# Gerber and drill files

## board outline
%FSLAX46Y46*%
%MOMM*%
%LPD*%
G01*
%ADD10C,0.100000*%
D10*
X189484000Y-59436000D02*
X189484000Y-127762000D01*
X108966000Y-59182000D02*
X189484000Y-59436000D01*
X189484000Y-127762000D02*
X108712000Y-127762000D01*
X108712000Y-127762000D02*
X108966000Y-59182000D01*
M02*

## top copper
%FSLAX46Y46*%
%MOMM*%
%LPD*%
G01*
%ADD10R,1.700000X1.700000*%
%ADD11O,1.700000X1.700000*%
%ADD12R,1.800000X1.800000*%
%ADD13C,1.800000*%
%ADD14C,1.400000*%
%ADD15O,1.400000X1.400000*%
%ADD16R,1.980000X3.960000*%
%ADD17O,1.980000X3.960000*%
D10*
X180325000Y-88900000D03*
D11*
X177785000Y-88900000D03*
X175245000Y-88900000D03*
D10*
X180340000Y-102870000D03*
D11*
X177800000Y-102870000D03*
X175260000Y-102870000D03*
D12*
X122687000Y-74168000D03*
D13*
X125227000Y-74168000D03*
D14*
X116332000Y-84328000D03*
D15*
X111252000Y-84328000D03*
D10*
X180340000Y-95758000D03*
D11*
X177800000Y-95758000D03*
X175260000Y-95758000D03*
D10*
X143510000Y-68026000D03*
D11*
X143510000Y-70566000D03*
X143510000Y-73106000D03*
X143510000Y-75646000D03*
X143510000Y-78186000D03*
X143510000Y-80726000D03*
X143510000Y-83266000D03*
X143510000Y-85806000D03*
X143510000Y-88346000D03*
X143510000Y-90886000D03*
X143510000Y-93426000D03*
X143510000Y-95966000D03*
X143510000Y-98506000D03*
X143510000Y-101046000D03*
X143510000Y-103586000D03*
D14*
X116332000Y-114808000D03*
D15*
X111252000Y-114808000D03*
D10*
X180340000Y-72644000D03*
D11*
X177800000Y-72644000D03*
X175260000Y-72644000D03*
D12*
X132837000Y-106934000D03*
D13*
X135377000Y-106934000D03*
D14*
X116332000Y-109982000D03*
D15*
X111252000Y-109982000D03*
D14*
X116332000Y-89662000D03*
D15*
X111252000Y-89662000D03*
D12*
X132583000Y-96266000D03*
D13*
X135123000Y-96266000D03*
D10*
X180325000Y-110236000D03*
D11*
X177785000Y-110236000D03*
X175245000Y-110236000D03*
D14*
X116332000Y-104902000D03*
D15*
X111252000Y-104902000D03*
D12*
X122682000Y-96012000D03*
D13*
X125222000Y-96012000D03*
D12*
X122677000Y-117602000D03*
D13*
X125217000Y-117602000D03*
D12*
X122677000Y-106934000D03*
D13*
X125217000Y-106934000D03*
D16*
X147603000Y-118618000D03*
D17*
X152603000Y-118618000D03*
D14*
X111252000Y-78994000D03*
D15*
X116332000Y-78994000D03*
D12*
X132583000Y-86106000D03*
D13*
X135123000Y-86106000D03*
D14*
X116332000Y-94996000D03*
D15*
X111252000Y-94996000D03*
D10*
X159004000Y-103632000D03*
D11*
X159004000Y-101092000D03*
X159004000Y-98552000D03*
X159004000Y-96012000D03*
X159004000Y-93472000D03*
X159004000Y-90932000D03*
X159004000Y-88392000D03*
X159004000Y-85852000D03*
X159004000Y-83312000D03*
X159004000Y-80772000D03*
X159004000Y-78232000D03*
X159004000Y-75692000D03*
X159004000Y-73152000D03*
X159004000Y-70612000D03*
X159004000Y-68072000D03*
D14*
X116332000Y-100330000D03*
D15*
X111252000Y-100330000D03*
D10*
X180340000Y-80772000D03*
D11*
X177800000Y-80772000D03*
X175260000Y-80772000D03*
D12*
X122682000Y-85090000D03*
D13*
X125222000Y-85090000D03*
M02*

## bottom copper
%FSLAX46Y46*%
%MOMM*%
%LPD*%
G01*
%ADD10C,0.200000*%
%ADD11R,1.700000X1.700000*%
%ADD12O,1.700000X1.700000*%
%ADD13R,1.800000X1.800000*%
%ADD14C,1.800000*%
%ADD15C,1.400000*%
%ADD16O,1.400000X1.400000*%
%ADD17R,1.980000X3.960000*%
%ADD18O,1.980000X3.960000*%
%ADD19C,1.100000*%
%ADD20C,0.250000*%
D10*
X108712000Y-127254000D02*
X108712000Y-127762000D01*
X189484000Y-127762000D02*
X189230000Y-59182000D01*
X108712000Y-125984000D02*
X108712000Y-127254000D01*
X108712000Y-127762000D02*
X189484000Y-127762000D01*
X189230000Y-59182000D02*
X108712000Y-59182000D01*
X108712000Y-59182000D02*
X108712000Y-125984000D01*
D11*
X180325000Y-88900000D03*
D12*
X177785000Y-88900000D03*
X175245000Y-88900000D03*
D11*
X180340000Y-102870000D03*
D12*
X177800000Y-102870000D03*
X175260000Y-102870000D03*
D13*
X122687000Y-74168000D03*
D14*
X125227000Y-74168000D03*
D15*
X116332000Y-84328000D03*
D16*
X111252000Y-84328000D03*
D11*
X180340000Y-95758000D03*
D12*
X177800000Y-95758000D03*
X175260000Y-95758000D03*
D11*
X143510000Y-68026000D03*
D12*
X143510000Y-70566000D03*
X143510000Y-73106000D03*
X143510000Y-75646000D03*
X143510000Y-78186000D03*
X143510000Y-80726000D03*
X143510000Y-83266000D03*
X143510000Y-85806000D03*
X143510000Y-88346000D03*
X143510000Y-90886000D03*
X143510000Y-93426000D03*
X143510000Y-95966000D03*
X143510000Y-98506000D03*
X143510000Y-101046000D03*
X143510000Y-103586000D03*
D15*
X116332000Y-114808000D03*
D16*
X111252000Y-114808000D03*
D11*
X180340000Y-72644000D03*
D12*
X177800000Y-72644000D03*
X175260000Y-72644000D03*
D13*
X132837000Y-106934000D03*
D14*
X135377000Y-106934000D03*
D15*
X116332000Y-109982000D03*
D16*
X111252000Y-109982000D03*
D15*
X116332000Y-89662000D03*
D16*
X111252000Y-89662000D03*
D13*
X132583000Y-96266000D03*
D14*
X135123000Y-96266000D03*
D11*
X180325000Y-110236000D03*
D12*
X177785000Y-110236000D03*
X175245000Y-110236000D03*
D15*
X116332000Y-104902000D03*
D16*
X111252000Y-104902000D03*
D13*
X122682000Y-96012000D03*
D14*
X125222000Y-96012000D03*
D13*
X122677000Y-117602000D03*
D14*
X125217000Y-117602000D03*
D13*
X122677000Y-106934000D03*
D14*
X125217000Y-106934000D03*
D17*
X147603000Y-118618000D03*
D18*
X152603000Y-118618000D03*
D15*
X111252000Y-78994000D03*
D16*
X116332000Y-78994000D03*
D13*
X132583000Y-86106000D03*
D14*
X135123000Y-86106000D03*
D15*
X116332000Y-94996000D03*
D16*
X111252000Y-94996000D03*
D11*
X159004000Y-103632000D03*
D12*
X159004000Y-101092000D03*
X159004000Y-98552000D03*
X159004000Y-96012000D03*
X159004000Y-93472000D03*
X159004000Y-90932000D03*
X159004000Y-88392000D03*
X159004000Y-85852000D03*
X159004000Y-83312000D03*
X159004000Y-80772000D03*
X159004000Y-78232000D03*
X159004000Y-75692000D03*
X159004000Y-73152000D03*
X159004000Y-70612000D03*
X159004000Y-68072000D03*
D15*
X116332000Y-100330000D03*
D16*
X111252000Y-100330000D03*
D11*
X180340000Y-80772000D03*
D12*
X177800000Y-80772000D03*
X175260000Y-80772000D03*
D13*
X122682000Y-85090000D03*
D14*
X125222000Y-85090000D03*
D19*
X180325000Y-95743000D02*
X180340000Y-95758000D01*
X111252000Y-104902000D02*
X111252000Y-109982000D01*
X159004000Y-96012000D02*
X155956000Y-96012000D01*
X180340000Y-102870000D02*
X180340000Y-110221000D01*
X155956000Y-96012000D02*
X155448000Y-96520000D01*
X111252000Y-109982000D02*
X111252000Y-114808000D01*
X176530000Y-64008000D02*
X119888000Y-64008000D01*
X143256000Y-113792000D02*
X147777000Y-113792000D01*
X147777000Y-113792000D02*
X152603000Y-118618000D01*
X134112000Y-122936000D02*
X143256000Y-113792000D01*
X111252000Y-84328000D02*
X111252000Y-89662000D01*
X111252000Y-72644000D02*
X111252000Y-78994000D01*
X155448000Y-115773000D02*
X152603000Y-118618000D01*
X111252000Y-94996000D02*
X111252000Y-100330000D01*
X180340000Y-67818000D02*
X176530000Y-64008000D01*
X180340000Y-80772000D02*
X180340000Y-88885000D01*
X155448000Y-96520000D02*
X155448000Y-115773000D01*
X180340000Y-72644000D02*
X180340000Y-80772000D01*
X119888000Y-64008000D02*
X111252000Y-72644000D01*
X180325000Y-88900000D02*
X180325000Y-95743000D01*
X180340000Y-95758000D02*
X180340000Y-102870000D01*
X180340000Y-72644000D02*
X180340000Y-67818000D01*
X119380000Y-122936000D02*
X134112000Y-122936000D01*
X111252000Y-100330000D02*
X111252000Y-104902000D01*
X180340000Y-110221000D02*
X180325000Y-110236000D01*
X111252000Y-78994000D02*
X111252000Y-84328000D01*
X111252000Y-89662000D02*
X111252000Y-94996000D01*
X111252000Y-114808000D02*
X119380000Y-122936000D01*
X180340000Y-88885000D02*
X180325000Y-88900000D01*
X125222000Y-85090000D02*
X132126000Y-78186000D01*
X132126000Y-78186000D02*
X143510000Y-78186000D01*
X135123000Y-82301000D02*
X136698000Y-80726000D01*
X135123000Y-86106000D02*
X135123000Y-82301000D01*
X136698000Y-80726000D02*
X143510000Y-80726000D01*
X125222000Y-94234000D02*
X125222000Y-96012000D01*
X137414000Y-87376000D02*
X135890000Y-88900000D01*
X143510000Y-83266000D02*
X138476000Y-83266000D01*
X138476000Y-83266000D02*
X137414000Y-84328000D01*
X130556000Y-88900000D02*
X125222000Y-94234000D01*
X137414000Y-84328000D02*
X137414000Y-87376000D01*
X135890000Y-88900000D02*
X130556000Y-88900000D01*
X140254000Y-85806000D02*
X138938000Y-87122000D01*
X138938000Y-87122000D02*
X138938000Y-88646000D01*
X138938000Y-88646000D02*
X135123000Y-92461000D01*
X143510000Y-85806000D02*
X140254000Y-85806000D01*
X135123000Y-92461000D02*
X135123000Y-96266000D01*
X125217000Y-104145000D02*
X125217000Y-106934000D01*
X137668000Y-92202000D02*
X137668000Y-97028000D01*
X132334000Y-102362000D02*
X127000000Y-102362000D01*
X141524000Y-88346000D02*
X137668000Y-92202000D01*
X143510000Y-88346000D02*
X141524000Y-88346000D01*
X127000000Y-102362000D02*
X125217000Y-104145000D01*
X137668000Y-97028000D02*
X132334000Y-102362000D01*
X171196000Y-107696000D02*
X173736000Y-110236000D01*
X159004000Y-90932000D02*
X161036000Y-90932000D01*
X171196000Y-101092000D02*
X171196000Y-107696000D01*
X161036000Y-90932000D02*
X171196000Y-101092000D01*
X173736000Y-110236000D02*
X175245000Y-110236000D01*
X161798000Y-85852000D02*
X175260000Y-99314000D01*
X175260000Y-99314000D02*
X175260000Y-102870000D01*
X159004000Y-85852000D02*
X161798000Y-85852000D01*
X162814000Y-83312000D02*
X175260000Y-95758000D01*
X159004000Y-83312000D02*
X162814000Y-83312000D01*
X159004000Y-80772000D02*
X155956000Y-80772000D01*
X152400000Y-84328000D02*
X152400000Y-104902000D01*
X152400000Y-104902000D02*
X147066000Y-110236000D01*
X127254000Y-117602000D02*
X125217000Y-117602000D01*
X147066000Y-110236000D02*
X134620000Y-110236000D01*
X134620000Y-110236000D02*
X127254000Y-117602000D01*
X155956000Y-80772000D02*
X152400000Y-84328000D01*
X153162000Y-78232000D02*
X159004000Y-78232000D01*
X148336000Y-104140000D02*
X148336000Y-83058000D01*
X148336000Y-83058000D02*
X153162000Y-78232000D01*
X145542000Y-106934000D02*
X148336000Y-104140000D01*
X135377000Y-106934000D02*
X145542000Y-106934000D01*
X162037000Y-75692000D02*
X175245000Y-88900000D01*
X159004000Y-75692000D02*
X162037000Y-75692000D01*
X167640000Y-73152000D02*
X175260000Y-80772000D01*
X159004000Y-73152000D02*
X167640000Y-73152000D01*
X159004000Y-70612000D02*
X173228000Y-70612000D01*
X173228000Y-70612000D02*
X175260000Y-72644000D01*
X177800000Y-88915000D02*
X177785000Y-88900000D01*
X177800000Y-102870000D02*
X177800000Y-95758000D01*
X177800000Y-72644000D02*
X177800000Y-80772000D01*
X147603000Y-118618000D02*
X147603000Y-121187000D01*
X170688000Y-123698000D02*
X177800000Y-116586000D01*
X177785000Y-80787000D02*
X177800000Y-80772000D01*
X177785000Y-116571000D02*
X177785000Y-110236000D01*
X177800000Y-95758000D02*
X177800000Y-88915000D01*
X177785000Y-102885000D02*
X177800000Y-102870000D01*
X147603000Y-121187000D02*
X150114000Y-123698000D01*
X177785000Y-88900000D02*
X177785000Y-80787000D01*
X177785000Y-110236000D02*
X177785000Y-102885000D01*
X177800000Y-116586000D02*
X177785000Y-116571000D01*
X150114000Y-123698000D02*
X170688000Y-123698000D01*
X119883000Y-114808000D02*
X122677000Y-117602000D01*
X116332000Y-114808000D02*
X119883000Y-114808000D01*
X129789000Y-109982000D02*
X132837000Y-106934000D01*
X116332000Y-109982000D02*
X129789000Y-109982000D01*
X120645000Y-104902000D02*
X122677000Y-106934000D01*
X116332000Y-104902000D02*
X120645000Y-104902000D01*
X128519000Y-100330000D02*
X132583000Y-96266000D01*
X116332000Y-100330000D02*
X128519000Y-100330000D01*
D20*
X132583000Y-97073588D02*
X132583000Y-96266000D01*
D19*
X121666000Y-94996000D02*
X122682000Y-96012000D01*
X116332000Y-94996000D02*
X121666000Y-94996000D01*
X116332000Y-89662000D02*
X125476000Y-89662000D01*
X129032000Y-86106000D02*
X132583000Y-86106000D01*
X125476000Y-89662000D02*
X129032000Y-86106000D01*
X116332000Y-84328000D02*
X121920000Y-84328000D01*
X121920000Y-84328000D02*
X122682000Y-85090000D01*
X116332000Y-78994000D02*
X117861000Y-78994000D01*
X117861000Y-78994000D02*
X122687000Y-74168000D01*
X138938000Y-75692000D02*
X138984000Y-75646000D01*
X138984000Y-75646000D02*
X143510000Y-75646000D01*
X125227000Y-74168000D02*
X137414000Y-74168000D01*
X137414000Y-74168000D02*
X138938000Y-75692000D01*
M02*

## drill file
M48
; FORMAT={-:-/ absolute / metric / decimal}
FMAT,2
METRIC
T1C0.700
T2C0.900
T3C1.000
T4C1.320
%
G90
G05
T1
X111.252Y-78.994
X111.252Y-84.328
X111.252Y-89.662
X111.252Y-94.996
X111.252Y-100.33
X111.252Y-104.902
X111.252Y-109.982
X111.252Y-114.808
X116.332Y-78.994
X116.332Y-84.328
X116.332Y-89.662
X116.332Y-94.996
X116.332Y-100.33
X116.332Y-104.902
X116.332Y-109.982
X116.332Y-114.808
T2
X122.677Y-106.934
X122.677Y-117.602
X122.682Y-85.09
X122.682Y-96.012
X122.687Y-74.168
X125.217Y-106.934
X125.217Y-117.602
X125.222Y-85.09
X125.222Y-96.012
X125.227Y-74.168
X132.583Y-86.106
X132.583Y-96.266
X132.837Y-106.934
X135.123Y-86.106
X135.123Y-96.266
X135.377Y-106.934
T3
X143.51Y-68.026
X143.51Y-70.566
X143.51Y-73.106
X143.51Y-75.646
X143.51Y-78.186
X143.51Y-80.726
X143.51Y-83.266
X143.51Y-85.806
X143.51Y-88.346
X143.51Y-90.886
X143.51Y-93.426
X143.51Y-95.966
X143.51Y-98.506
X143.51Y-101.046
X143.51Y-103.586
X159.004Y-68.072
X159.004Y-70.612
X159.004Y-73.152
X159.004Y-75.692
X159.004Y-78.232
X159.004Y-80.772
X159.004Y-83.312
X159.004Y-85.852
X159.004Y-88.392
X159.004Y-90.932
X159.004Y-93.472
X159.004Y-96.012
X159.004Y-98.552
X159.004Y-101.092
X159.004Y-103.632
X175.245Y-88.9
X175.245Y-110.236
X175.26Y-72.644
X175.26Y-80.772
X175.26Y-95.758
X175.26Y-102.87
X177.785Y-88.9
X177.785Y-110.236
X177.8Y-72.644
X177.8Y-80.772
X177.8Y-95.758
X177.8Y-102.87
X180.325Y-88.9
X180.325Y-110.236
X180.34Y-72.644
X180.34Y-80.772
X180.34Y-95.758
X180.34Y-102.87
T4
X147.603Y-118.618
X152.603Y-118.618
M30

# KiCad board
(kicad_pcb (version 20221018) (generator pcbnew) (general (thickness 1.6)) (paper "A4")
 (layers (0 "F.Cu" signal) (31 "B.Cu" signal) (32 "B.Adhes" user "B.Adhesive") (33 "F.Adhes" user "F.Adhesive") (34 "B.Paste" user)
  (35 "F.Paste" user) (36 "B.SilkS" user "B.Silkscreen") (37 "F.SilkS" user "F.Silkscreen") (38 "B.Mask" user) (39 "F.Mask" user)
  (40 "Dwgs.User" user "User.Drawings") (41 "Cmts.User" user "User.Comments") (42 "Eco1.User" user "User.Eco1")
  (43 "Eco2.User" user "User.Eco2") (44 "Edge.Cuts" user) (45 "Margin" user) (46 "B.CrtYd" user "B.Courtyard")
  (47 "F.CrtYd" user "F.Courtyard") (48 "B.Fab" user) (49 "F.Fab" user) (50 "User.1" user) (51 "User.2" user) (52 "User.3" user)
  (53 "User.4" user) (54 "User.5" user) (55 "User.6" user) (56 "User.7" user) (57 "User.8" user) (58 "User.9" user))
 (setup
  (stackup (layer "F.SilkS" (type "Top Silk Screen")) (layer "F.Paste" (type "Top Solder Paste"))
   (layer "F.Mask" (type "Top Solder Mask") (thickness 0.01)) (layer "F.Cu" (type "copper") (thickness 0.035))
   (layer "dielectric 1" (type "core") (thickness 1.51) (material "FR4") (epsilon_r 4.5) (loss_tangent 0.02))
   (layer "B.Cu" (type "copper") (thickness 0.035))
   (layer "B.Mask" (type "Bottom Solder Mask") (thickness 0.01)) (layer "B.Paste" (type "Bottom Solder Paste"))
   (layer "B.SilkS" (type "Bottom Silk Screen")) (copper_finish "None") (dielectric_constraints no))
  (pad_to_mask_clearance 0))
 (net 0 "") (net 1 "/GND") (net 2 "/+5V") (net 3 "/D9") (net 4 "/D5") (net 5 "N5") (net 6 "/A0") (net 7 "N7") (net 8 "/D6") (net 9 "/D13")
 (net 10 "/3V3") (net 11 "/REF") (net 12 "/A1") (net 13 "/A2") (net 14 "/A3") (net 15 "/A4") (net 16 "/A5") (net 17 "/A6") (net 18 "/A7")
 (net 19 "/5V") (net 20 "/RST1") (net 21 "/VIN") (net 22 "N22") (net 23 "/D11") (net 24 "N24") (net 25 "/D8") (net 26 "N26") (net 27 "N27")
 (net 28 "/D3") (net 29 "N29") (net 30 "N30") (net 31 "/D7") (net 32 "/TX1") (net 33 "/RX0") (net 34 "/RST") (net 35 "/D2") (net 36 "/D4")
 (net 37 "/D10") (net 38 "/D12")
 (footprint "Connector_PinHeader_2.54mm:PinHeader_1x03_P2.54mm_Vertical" (layer "F.Cu") (at 180.325 88.9 -90)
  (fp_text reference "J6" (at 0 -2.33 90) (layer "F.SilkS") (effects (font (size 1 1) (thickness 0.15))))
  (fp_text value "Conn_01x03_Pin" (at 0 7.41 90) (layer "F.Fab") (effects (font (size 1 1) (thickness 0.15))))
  (pad "1" thru_hole rect (at 0 0 270) (size 1.7 1.7) (drill 1) (layers "*.Cu" "*.Mask") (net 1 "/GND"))
  (pad "2" thru_hole oval (at 0 2.54 270) (size 1.7 1.7) (drill 1) (layers "*.Cu" "*.Mask") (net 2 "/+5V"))
  (pad "3" thru_hole oval (at 0 5.08 270) (size 1.7 1.7) (drill 1) (layers "*.Cu" "*.Mask") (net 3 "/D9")))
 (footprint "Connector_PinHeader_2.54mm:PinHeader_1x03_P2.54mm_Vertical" (layer "F.Cu") (at 180.34 102.87 -90)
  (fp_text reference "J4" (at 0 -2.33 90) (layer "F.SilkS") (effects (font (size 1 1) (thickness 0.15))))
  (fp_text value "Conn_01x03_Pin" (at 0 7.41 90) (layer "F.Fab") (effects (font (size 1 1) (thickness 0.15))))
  (pad "1" thru_hole rect (at 0 0 270) (size 1.7 1.7) (drill 1) (layers "*.Cu" "*.Mask") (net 1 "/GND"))
  (pad "2" thru_hole oval (at 0 2.54 270) (size 1.7 1.7) (drill 1) (layers "*.Cu" "*.Mask") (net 2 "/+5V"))
  (pad "3" thru_hole oval (at 0 5.08 270) (size 1.7 1.7) (drill 1) (layers "*.Cu" "*.Mask") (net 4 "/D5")))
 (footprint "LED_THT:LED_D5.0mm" (layer "F.Cu") (at 122.687 74.168)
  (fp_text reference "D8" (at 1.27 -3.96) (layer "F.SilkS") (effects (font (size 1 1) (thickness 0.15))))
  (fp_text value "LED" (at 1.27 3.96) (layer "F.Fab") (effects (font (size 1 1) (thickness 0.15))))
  (pad "1" thru_hole rect (at 0 0) (size 1.8 1.8) (drill 0.9) (layers "*.Cu" "*.Mask") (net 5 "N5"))
  (pad "2" thru_hole circle (at 2.54 0) (size 1.8 1.8) (drill 0.9) (layers "*.Cu" "*.Mask") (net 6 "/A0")))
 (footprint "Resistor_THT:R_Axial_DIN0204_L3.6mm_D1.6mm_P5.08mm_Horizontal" (layer "F.Cu") (at 116.332 84.328 180)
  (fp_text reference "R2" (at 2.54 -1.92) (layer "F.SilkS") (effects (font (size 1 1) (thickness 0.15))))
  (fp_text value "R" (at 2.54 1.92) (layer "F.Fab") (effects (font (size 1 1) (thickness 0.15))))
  (pad "1" thru_hole circle (at 0 0 180) (size 1.4 1.4) (drill 0.7) (layers "*.Cu" "*.Mask") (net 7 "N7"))
  (pad "2" thru_hole oval (at 5.08 0 180) (size 1.4 1.4) (drill 0.7) (layers "*.Cu" "*.Mask") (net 1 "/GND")))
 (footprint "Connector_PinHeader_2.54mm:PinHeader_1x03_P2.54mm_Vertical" (layer "F.Cu") (at 180.34 95.758 -90)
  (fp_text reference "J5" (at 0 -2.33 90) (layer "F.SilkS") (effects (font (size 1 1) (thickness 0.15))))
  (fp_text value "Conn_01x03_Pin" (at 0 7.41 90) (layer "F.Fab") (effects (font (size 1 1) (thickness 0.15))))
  (pad "1" thru_hole rect (at 0 0 270) (size 1.7 1.7) (drill 1) (layers "*.Cu" "*.Mask") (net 1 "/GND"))
  (pad "2" thru_hole oval (at 0 2.54 270) (size 1.7 1.7) (drill 1) (layers "*.Cu" "*.Mask") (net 2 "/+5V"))
  (pad "3" thru_hole oval (at 0 5.08 270) (size 1.7 1.7) (drill 1) (layers "*.Cu" "*.Mask") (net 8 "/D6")))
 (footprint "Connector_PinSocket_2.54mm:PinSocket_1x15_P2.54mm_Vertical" (layer "F.Cu") (at 143.51 68.026)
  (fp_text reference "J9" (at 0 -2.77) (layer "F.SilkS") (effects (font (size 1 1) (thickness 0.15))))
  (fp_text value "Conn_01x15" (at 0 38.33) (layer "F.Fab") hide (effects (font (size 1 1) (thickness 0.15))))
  (pad "1" thru_hole rect (at 0 0) (size 1.7 1.7) (drill 1) (layers "*.Cu" "*.Mask") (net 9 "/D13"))
  (pad "2" thru_hole oval (at 0 2.54) (size 1.7 1.7) (drill 1) (layers "*.Cu" "*.Mask") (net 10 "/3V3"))
  (pad "3" thru_hole oval (at 0 5.08) (size 1.7 1.7) (drill 1) (layers "*.Cu" "*.Mask") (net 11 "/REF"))
  (pad "4" thru_hole oval (at 0 7.62) (size 1.7 1.7) (drill 1) (layers "*.Cu" "*.Mask") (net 6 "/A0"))
  (pad "5" thru_hole oval (at 0 10.16) (size 1.7 1.7) (drill 1) (layers "*.Cu" "*.Mask") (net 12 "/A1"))
  (pad "6" thru_hole oval (at 0 12.7) (size 1.7 1.7) (drill 1) (layers "*.Cu" "*.Mask") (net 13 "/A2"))
  (pad "7" thru_hole oval (at 0 15.24) (size 1.7 1.7) (drill 1) (layers "*.Cu" "*.Mask") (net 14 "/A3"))
  (pad "8" thru_hole oval (at 0 17.78) (size 1.7 1.7) (drill 1) (layers "*.Cu" "*.Mask") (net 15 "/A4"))
  (pad "9" thru_hole oval (at 0 20.32) (size 1.7 1.7) (drill 1) (layers "*.Cu" "*.Mask") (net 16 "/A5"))
  (pad "10" thru_hole oval (at 0 22.86) (size 1.7 1.7) (drill 1) (layers "*.Cu" "*.Mask") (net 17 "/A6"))
  (pad "11" thru_hole oval (at 0 25.4) (size 1.7 1.7) (drill 1) (layers "*.Cu" "*.Mask") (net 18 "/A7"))
  (pad "12" thru_hole oval (at 0 27.94) (size 1.7 1.7) (drill 1) (layers "*.Cu" "*.Mask") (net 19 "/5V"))
  (pad "13" thru_hole oval (at 0 30.48) (size 1.7 1.7) (drill 1) (layers "*.Cu" "*.Mask") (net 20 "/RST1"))
  (pad "14" thru_hole oval (at 0 33.02) (size 1.7 1.7) (drill 1) (layers "*.Cu" "*.Mask") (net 1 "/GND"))
  (pad "15" thru_hole oval (at 0 35.56) (size 1.7 1.7) (drill 1) (layers "*.Cu" "*.Mask") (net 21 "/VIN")))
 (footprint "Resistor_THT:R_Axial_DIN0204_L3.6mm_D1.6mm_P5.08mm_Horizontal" (layer "F.Cu") (at 116.332 114.808 180)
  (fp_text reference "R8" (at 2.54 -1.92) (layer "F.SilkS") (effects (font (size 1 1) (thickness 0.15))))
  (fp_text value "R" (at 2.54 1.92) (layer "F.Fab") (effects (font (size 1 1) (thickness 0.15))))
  (pad "1" thru_hole circle (at 0 0 180) (size 1.4 1.4) (drill 0.7) (layers "*.Cu" "*.Mask") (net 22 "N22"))
  (pad "2" thru_hole oval (at 5.08 0 180) (size 1.4 1.4) (drill 0.7) (layers "*.Cu" "*.Mask") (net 1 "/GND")))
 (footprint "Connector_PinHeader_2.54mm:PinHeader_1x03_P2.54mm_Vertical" (layer "F.Cu") (at 180.34 72.644 -90)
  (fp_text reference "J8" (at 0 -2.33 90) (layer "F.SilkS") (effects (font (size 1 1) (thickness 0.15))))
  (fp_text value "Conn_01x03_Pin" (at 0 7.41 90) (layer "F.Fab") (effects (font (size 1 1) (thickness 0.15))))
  (pad "1" thru_hole rect (at 0 0 270) (size 1.7 1.7) (drill 1) (layers "*.Cu" "*.Mask") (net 1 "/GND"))
  (pad "2" thru_hole oval (at 0 2.54 270) (size 1.7 1.7) (drill 1) (layers "*.Cu" "*.Mask") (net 2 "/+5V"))
  (pad "3" thru_hole oval (at 0 5.08 270) (size 1.7 1.7) (drill 1) (layers "*.Cu" "*.Mask") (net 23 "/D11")))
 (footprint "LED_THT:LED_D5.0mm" (layer "F.Cu") (at 132.837 106.934)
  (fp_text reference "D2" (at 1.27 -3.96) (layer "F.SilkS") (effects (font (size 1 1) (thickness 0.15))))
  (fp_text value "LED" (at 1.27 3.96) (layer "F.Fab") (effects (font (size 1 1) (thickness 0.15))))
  (pad "1" thru_hole rect (at 0 0) (size 1.8 1.8) (drill 0.9) (layers "*.Cu" "*.Mask") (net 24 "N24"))
  (pad "2" thru_hole circle (at 2.54 0) (size 1.8 1.8) (drill 0.9) (layers "*.Cu" "*.Mask") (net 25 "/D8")))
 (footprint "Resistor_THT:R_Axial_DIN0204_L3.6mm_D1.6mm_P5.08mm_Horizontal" (layer "F.Cu") (at 116.332 109.982 180)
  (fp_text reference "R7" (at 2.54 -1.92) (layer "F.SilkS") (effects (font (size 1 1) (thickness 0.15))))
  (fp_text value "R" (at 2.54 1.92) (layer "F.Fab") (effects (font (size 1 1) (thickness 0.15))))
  (pad "1" thru_hole circle (at 0 0 180) (size 1.4 1.4) (drill 0.7) (layers "*.Cu" "*.Mask") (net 24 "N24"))
  (pad "2" thru_hole oval (at 5.08 0 180) (size 1.4 1.4) (drill 0.7) (layers "*.Cu" "*.Mask") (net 1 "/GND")))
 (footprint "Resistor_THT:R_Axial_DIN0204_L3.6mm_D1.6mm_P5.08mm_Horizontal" (layer "F.Cu") (at 116.332 89.662 180)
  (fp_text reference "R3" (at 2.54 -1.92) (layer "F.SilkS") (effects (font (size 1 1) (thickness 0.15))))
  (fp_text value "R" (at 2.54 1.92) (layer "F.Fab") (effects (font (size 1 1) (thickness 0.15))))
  (pad "1" thru_hole circle (at 0 0 180) (size 1.4 1.4) (drill 0.7) (layers "*.Cu" "*.Mask") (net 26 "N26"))
  (pad "2" thru_hole oval (at 5.08 0 180) (size 1.4 1.4) (drill 0.7) (layers "*.Cu" "*.Mask") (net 1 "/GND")))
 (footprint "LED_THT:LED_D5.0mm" (layer "F.Cu") (at 132.583 96.266)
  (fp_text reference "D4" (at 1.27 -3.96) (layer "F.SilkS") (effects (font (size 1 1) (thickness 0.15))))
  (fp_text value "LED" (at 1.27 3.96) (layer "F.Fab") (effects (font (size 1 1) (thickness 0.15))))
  (pad "1" thru_hole rect (at 0 0) (size 1.8 1.8) (drill 0.9) (layers "*.Cu" "*.Mask") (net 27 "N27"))
  (pad "2" thru_hole circle (at 2.54 0) (size 1.8 1.8) (drill 0.9) (layers "*.Cu" "*.Mask") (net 15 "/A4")))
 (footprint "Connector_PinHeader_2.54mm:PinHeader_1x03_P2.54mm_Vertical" (layer "F.Cu") (at 180.325 110.236 -90)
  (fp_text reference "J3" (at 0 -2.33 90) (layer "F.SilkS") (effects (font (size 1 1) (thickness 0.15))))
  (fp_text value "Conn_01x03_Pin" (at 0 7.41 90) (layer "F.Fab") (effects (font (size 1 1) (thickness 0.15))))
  (pad "1" thru_hole rect (at 0 0 270) (size 1.7 1.7) (drill 1) (layers "*.Cu" "*.Mask") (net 1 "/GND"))
  (pad "2" thru_hole oval (at 0 2.54 270) (size 1.7 1.7) (drill 1) (layers "*.Cu" "*.Mask") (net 2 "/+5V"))
  (pad "3" thru_hole oval (at 0 5.08 270) (size 1.7 1.7) (drill 1) (layers "*.Cu" "*.Mask") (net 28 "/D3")))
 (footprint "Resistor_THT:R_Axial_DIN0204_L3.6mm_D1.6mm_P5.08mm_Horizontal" (layer "F.Cu") (at 116.332 104.902 180)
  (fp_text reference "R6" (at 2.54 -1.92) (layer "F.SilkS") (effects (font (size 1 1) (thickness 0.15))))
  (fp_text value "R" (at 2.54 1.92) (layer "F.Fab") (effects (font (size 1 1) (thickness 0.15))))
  (pad "1" thru_hole circle (at 0 0 180) (size 1.4 1.4) (drill 0.7) (layers "*.Cu" "*.Mask") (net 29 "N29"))
  (pad "2" thru_hole oval (at 5.08 0 180) (size 1.4 1.4) (drill 0.7) (layers "*.Cu" "*.Mask") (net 1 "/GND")))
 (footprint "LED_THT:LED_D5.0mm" (layer "F.Cu") (at 122.682 96.012)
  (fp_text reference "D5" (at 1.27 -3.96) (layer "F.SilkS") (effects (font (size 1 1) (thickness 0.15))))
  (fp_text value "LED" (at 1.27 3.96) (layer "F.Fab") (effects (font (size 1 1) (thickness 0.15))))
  (pad "1" thru_hole rect (at 0 0) (size 1.8 1.8) (drill 0.9) (layers "*.Cu" "*.Mask") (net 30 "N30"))
  (pad "2" thru_hole circle (at 2.54 0) (size 1.8 1.8) (drill 0.9) (layers "*.Cu" "*.Mask") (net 14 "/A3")))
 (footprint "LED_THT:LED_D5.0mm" (layer "F.Cu") (at 122.677 117.602)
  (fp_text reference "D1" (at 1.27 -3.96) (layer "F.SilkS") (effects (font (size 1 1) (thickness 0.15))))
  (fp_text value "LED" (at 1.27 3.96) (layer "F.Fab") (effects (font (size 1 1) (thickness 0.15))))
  (pad "1" thru_hole rect (at 0 0) (size 1.8 1.8) (drill 0.9) (layers "*.Cu" "*.Mask") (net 22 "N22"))
  (pad "2" thru_hole circle (at 2.54 0) (size 1.8 1.8) (drill 0.9) (layers "*.Cu" "*.Mask") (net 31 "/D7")))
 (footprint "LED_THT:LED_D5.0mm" (layer "F.Cu") (at 122.677 106.934)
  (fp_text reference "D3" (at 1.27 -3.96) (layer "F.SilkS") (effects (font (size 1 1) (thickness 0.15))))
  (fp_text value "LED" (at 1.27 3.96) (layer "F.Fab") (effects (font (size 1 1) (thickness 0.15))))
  (pad "1" thru_hole rect (at 0 0) (size 1.8 1.8) (drill 0.9) (layers "*.Cu" "*.Mask") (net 29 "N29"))
  (pad "2" thru_hole circle (at 2.54 0) (size 1.8 1.8) (drill 0.9) (layers "*.Cu" "*.Mask") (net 16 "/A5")))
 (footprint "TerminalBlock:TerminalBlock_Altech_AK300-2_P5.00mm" (layer "F.Cu") (at 147.603 118.618)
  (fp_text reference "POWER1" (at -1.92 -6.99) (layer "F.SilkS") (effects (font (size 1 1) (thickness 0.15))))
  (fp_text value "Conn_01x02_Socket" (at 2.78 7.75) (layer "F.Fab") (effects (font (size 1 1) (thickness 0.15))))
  (pad "1" thru_hole rect (at 0 0) (size 1.98 3.96) (drill 1.32) (layers "*.Cu" "*.Mask") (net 2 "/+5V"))
  (pad "2" thru_hole oval (at 5 0) (size 1.98 3.96) (drill 1.32) (layers "*.Cu" "*.Mask") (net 1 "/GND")))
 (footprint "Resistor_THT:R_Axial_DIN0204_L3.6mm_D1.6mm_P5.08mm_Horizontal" (layer "F.Cu") (at 111.252 78.994)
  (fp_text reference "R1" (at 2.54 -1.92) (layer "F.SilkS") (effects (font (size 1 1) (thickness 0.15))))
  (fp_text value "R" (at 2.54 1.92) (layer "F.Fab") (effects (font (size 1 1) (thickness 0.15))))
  (pad "1" thru_hole circle (at 0 0) (size 1.4 1.4) (drill 0.7) (layers "*.Cu" "*.Mask") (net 1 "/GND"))
  (pad "2" thru_hole oval (at 5.08 0) (size 1.4 1.4) (drill 0.7) (layers "*.Cu" "*.Mask") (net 5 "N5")))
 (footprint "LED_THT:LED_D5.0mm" (layer "F.Cu") (at 132.583 86.106)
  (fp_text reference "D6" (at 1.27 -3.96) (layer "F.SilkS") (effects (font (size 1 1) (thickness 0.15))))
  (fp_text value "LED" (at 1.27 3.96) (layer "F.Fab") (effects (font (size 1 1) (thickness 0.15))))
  (pad "1" thru_hole rect (at 0 0) (size 1.8 1.8) (drill 0.9) (layers "*.Cu" "*.Mask") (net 26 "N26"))
  (pad "2" thru_hole circle (at 2.54 0) (size 1.8 1.8) (drill 0.9) (layers "*.Cu" "*.Mask") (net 13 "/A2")))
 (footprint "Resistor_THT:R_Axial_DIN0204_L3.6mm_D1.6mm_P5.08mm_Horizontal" (layer "F.Cu") (at 116.332 94.996 180)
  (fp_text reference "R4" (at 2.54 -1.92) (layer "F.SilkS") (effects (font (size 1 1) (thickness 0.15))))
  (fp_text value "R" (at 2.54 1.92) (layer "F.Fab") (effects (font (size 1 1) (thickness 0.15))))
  (pad "1" thru_hole circle (at 0 0 180) (size 1.4 1.4) (drill 0.7) (layers "*.Cu" "*.Mask") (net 30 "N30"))
  (pad "2" thru_hole oval (at 5.08 0 180) (size 1.4 1.4) (drill 0.7) (layers "*.Cu" "*.Mask") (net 1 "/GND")))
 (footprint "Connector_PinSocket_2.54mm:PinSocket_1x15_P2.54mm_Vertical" (layer "F.Cu") (at 159.004 103.632 180)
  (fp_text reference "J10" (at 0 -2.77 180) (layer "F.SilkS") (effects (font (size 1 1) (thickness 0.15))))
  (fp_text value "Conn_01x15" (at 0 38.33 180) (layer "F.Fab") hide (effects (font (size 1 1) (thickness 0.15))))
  (pad "1" thru_hole rect (at 0 0 180) (size 1.7 1.7) (drill 1) (layers "*.Cu" "*.Mask") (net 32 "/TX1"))
  (pad "2" thru_hole oval (at 0 2.54 180) (size 1.7 1.7) (drill 1) (layers "*.Cu" "*.Mask") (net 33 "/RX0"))
  (pad "3" thru_hole oval (at 0 5.08 180) (size 1.7 1.7) (drill 1) (layers "*.Cu" "*.Mask") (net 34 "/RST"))
  (pad "4" thru_hole oval (at 0 7.62 180) (size 1.7 1.7) (drill 1) (layers "*.Cu" "*.Mask") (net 1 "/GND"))
  (pad "5" thru_hole oval (at 0 10.16 180) (size 1.7 1.7) (drill 1) (layers "*.Cu" "*.Mask") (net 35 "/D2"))
  (pad "6" thru_hole oval (at 0 12.7 180) (size 1.7 1.7) (drill 1) (layers "*.Cu" "*.Mask") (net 28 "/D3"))
  (pad "7" thru_hole oval (at 0 15.24 180) (size 1.7 1.7) (drill 1) (layers "*.Cu" "*.Mask") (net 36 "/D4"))
  (pad "8" thru_hole oval (at 0 17.78 180) (size 1.7 1.7) (drill 1) (layers "*.Cu" "*.Mask") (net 4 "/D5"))
  (pad "9" thru_hole oval (at 0 20.32 180) (size 1.7 1.7) (drill 1) (layers "*.Cu" "*.Mask") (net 8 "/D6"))
  (pad "10" thru_hole oval (at 0 22.86 180) (size 1.7 1.7) (drill 1) (layers "*.Cu" "*.Mask") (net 31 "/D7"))
  (pad "11" thru_hole oval (at 0 25.4 180) (size 1.7 1.7) (drill 1) (layers "*.Cu" "*.Mask") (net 25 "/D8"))
  (pad "12" thru_hole oval (at 0 27.94 180) (size 1.7 1.7) (drill 1) (layers "*.Cu" "*.Mask") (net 3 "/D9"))
  (pad "13" thru_hole oval (at 0 30.48 180) (size 1.7 1.7) (drill 1) (layers "*.Cu" "*.Mask") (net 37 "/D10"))
  (pad "14" thru_hole oval (at 0 33.02 180) (size 1.7 1.7) (drill 1) (layers "*.Cu" "*.Mask") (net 23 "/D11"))
  (pad "15" thru_hole oval (at 0 35.56 180) (size 1.7 1.7) (drill 1) (layers "*.Cu" "*.Mask") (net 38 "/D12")))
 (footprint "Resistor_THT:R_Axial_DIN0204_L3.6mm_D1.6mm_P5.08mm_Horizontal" (layer "F.Cu") (at 116.332 100.33 180)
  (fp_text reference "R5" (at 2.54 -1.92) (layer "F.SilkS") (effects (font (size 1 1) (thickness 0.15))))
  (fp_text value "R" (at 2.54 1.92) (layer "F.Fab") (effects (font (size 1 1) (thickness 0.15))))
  (pad "1" thru_hole circle (at 0 0 180) (size 1.4 1.4) (drill 0.7) (layers "*.Cu" "*.Mask") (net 27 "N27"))
  (pad "2" thru_hole oval (at 5.08 0 180) (size 1.4 1.4) (drill 0.7) (layers "*.Cu" "*.Mask") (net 1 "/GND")))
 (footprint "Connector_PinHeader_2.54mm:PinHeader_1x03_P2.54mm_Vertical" (layer "F.Cu") (at 180.34 80.772 -90)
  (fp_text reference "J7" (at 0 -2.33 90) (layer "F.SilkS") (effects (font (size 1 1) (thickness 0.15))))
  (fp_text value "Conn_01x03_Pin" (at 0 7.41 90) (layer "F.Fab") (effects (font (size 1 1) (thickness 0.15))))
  (pad "1" thru_hole rect (at 0 0 270) (size 1.7 1.7) (drill 1) (layers "*.Cu" "*.Mask") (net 1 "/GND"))
  (pad "2" thru_hole oval (at 0 2.54 270) (size 1.7 1.7) (drill 1) (layers "*.Cu" "*.Mask") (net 2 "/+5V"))
  (pad "3" thru_hole oval (at 0 5.08 270) (size 1.7 1.7) (drill 1) (layers "*.Cu" "*.Mask") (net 37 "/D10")))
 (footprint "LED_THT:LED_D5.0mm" (layer "F.Cu") (at 122.682 85.09)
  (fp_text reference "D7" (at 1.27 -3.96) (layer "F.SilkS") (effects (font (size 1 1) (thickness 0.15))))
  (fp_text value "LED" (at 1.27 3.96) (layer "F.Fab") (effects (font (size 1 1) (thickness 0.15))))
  (pad "1" thru_hole rect (at 0 0) (size 1.8 1.8) (drill 0.9) (layers "*.Cu" "*.Mask") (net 7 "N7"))
  (pad "2" thru_hole circle (at 2.54 0) (size 1.8 1.8) (drill 0.9) (layers "*.Cu" "*.Mask") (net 12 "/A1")))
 (gr_line (start 108.712 127.254) (end 108.712 127.762) (stroke (width 0.2) (type default)) (layer "B.Cu"))
 (gr_line (start 189.484 127.762) (end 189.23 59.182) (stroke (width 0.2) (type default)) (layer "B.Cu"))
 (gr_line (start 108.712 125.984) (end 108.712 127.254) (stroke (width 0.2) (type default)) (layer "B.Cu"))
 (gr_line (start 108.712 127.762) (end 189.484 127.762) (stroke (width 0.2) (type default)) (layer "B.Cu"))
 (gr_line (start 189.23 59.182) (end 108.712 59.182) (stroke (width 0.2) (type default)) (layer "B.Cu"))
 (gr_line (start 108.712 59.182) (end 108.712 125.984) (stroke (width 0.2) (type default)) (layer "B.Cu"))
 (gr_line (start 189.484 59.436) (end 189.484 127.762) (stroke (width 0.1) (type default)) (layer "Edge.Cuts"))
 (gr_line (start 108.966 59.182) (end 189.484 59.436) (stroke (width 0.1) (type default)) (layer "Edge.Cuts"))
 (gr_line (start 189.484 127.762) (end 108.712 127.762) (stroke (width 0.1) (type default)) (layer "Edge.Cuts"))
 (gr_line (start 108.712 127.762) (end 108.966 59.182) (stroke (width 0.1) (type default)) (layer "Edge.Cuts"))
 (segment (start 180.325 95.743) (end 180.34 95.758) (width 1.1) (layer "B.Cu") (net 1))
 (segment (start 111.252 104.902) (end 111.252 109.982) (width 1.1) (layer "B.Cu") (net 1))
 (segment (start 159.004 96.012) (end 155.956 96.012) (width 1.1) (layer "B.Cu") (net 1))
 (segment (start 180.34 102.87) (end 180.34 110.221) (width 1.1) (layer "B.Cu") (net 1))
 (segment (start 155.956 96.012) (end 155.448 96.52) (width 1.1) (layer "B.Cu") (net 1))
 (segment (start 111.252 109.982) (end 111.252 114.808) (width 1.1) (layer "B.Cu") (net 1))
 (segment (start 176.53 64.008) (end 119.888 64.008) (width 1.1) (layer "B.Cu") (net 1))
 (segment (start 143.256 113.792) (end 147.777 113.792) (width 1.1) (layer "B.Cu") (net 1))
 (segment (start 147.777 113.792) (end 152.603 118.618) (width 1.1) (layer "B.Cu") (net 1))
 (segment (start 134.112 122.936) (end 143.256 113.792) (width 1.1) (layer "B.Cu") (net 1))
 (segment (start 111.252 84.328) (end 111.252 89.662) (width 1.1) (layer "B.Cu") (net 1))
 (segment (start 111.252 72.644) (end 111.252 78.994) (width 1.1) (layer "B.Cu") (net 1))
 (segment (start 155.448 115.773) (end 152.603 118.618) (width 1.1) (layer "B.Cu") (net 1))
 (segment (start 111.252 94.996) (end 111.252 100.33) (width 1.1) (layer "B.Cu") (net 1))
 (segment (start 180.34 67.818) (end 176.53 64.008) (width 1.1) (layer "B.Cu") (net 1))
 (segment (start 180.34 80.772) (end 180.34 88.885) (width 1.1) (layer "B.Cu") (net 1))
 (segment (start 155.448 96.52) (end 155.448 115.773) (width 1.1) (layer "B.Cu") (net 1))
 (segment (start 180.34 72.644) (end 180.34 80.772) (width 1.1) (layer "B.Cu") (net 1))
 (segment (start 119.888 64.008) (end 111.252 72.644) (width 1.1) (layer "B.Cu") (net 1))
 (segment (start 180.325 88.9) (end 180.325 95.743) (width 1.1) (layer "B.Cu") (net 1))
 (segment (start 180.34 95.758) (end 180.34 102.87) (width 1.1) (layer "B.Cu") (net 1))
 (segment (start 180.34 72.644) (end 180.34 67.818) (width 1.1) (layer "B.Cu") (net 1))
 (segment (start 119.38 122.936) (end 134.112 122.936) (width 1.1) (layer "B.Cu") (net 1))
 (segment (start 111.252 100.33) (end 111.252 104.902) (width 1.1) (layer "B.Cu") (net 1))
 (segment (start 180.34 110.221) (end 180.325 110.236) (width 1.1) (layer "B.Cu") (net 1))
 (segment (start 111.252 78.994) (end 111.252 84.328) (width 1.1) (layer "B.Cu") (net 1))
 (segment (start 111.252 89.662) (end 111.252 94.996) (width 1.1) (layer "B.Cu") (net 1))
 (segment (start 111.252 114.808) (end 119.38 122.936) (width 1.1) (layer "B.Cu") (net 1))
 (segment (start 180.34 88.885) (end 180.325 88.9) (width 1.1) (layer "B.Cu") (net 1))
 (segment (start 125.222 85.09) (end 132.126 78.186) (width 1.1) (layer "B.Cu") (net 12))
 (segment (start 132.126 78.186) (end 143.51 78.186) (width 1.1) (layer "B.Cu") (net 12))
 (segment (start 135.123 82.301) (end 136.698 80.726) (width 1.1) (layer "B.Cu") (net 13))
 (segment (start 135.123 86.106) (end 135.123 82.301) (width 1.1) (layer "B.Cu") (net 13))
 (segment (start 136.698 80.726) (end 143.51 80.726) (width 1.1) (layer "B.Cu") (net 13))
 (segment (start 125.222 94.234) (end 125.222 96.012) (width 1.1) (layer "B.Cu") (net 14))
 (segment (start 137.414 87.376) (end 135.89 88.9) (width 1.1) (layer "B.Cu") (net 14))
 (segment (start 143.51 83.266) (end 138.476 83.266) (width 1.1) (layer "B.Cu") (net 14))
 (segment (start 138.476 83.266) (end 137.414 84.328) (width 1.1) (layer "B.Cu") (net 14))
 (segment (start 130.556 88.9) (end 125.222 94.234) (width 1.1) (layer "B.Cu") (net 14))
 (segment (start 137.414 84.328) (end 137.414 87.376) (width 1.1) (layer "B.Cu") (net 14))
 (segment (start 135.89 88.9) (end 130.556 88.9) (width 1.1) (layer "B.Cu") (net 14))
 (segment (start 140.254 85.806) (end 138.938 87.122) (width 1.1) (layer "B.Cu") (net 15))
 (segment (start 138.938 87.122) (end 138.938 88.646) (width 1.1) (layer "B.Cu") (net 15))
 (segment (start 138.938 88.646) (end 135.123 92.461) (width 1.1) (layer "B.Cu") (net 15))
 (segment (start 143.51 85.806) (end 140.254 85.806) (width 1.1) (layer "B.Cu") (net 15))
 (segment (start 135.123 92.461) (end 135.123 96.266) (width 1.1) (layer "B.Cu") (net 15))
 (segment (start 125.217 104.145) (end 125.217 106.934) (width 1.1) (layer "B.Cu") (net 16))
 (segment (start 137.668 92.202) (end 137.668 97.028) (width 1.1) (layer "B.Cu") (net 16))
 (segment (start 132.334 102.362) (end 127 102.362) (width 1.1) (layer "B.Cu") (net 16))
 (segment (start 141.524 88.346) (end 137.668 92.202) (width 1.1) (layer "B.Cu") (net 16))
 (segment (start 143.51 88.346) (end 141.524 88.346) (width 1.1) (layer "B.Cu") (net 16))
 (segment (start 127 102.362) (end 125.217 104.145) (width 1.1) (layer "B.Cu") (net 16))
 (segment (start 137.668 97.028) (end 132.334 102.362) (width 1.1) (layer "B.Cu") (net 16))
 (segment (start 171.196 107.696) (end 173.736 110.236) (width 1.1) (layer "B.Cu") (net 28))
 (segment (start 159.004 90.932) (end 161.036 90.932) (width 1.1) (layer "B.Cu") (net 28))
 (segment (start 171.196 101.092) (end 171.196 107.696) (width 1.1) (layer "B.Cu") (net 28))
 (segment (start 161.036 90.932) (end 171.196 101.092) (width 1.1) (layer "B.Cu") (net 28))
 (segment (start 173.736 110.236) (end 175.245 110.236) (width 1.1) (layer "B.Cu") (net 28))
 (segment (start 161.798 85.852) (end 175.26 99.314) (width 1.1) (layer "B.Cu") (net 4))
 (segment (start 175.26 99.314) (end 175.26 102.87) (width 1.1) (layer "B.Cu") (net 4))
 (segment (start 159.004 85.852) (end 161.798 85.852) (width 1.1) (layer "B.Cu") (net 4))
 (segment (start 162.814 83.312) (end 175.26 95.758) (width 1.1) (layer "B.Cu") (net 8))
 (segment (start 159.004 83.312) (end 162.814 83.312) (width 1.1) (layer "B.Cu") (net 8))
 (segment (start 159.004 80.772) (end 155.956 80.772) (width 1.1) (layer "B.Cu") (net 31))
 (segment (start 152.4 84.328) (end 152.4 104.902) (width 1.1) (layer "B.Cu") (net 31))
 (segment (start 152.4 104.902) (end 147.066 110.236) (width 1.1) (layer "B.Cu") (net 31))
 (segment (start 127.254 117.602) (end 125.217 117.602) (width 1.1) (layer "B.Cu") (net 31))
 (segment (start 147.066 110.236) (end 134.62 110.236) (width 1.1) (layer "B.Cu") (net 31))
 (segment (start 134.62 110.236) (end 127.254 117.602) (width 1.1) (layer "B.Cu") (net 31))
 (segment (start 155.956 80.772) (end 152.4 84.328) (width 1.1) (layer "B.Cu") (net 31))
 (segment (start 153.162 78.232) (end 159.004 78.232) (width 1.1) (layer "B.Cu") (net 25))
 (segment (start 148.336 104.14) (end 148.336 83.058) (width 1.1) (layer "B.Cu") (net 25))
 (segment (start 148.336 83.058) (end 153.162 78.232) (width 1.1) (layer "B.Cu") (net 25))
 (segment (start 145.542 106.934) (end 148.336 104.14) (width 1.1) (layer "B.Cu") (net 25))
 (segment (start 135.377 106.934) (end 145.542 106.934) (width 1.1) (layer "B.Cu") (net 25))
 (segment (start 162.037 75.692) (end 175.245 88.9) (width 1.1) (layer "B.Cu") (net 3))
 (segment (start 159.004 75.692) (end 162.037 75.692) (width 1.1) (layer "B.Cu") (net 3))
 (segment (start 167.64 73.152) (end 175.26 80.772) (width 1.1) (layer "B.Cu") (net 37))
 (segment (start 159.004 73.152) (end 167.64 73.152) (width 1.1) (layer "B.Cu") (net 37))
 (segment (start 159.004 70.612) (end 173.228 70.612) (width 1.1) (layer "B.Cu") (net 23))
 (segment (start 173.228 70.612) (end 175.26 72.644) (width 1.1) (layer "B.Cu") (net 23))
 (segment (start 177.8 88.915) (end 177.785 88.9) (width 1.1) (layer "B.Cu") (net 2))
 (segment (start 177.8 102.87) (end 177.8 95.758) (width 1.1) (layer "B.Cu") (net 2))
 (segment (start 177.8 72.644) (end 177.8 80.772) (width 1.1) (layer "B.Cu") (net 2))
 (segment (start 147.603 118.618) (end 147.603 121.187) (width 1.1) (layer "B.Cu") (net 2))
 (segment (start 170.688 123.698) (end 177.8 116.586) (width 1.1) (layer "B.Cu") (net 2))
 (segment (start 177.785 80.787) (end 177.8 80.772) (width 1.1) (layer "B.Cu") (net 2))
 (segment (start 177.785 116.571) (end 177.785 110.236) (width 1.1) (layer "B.Cu") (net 2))
 (segment (start 177.8 95.758) (end 177.8 88.915) (width 1.1) (layer "B.Cu") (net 2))
 (segment (start 177.785 102.885) (end 177.8 102.87) (width 1.1) (layer "B.Cu") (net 2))
 (segment (start 147.603 121.187) (end 150.114 123.698) (width 1.1) (layer "B.Cu") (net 2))
 (segment (start 177.785 88.9) (end 177.785 80.787) (width 1.1) (layer "B.Cu") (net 2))
 (segment (start 177.785 110.236) (end 177.785 102.885) (width 1.1) (layer "B.Cu") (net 2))
 (segment (start 177.8 116.586) (end 177.785 116.571) (width 1.1) (layer "B.Cu") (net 2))
 (segment (start 150.114 123.698) (end 170.688 123.698) (width 1.1) (layer "B.Cu") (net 2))
 (segment (start 119.883 114.808) (end 122.677 117.602) (width 1.1) (layer "B.Cu") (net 22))
 (segment (start 116.332 114.808) (end 119.883 114.808) (width 1.1) (layer "B.Cu") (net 22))
 (segment (start 129.789 109.982) (end 132.837 106.934) (width 1.1) (layer "B.Cu") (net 24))
 (segment (start 116.332 109.982) (end 129.789 109.982) (width 1.1) (layer "B.Cu") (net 24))
 (segment (start 120.645 104.902) (end 122.677 106.934) (width 1.1) (layer "B.Cu") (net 29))
 (segment (start 116.332 104.902) (end 120.645 104.902) (width 1.1) (layer "B.Cu") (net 29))
 (segment (start 128.519 100.33) (end 132.583 96.266) (width 1.1) (layer "B.Cu") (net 27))
 (segment (start 116.332 100.33) (end 128.519 100.33) (width 1.1) (layer "B.Cu") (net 27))
 (segment (start 132.583 97.073588) (end 132.583 96.266) (width 0.25) (layer "B.Cu") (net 27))
 (segment (start 121.666 94.996) (end 122.682 96.012) (width 1.1) (layer "B.Cu") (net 30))
 (segment (start 116.332 94.996) (end 121.666 94.996) (width 1.1) (layer "B.Cu") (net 30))
 (segment (start 116.332 89.662) (end 125.476 89.662) (width 1.1) (layer "B.Cu") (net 26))
 (segment (start 129.032 86.106) (end 132.583 86.106) (width 1.1) (layer "B.Cu") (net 26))
 (segment (start 125.476 89.662) (end 129.032 86.106) (width 1.1) (layer "B.Cu") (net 26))
 (segment (start 116.332 84.328) (end 121.92 84.328) (width 1.1) (layer "B.Cu") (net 7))
 (segment (start 121.92 84.328) (end 122.682 85.09) (width 1.1) (layer "B.Cu") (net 7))
 (segment (start 116.332 78.994) (end 117.861 78.994) (width 1.1) (layer "B.Cu") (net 5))
 (segment (start 117.861 78.994) (end 122.687 74.168) (width 1.1) (layer "B.Cu") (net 5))
 (segment (start 138.938 75.692) (end 138.984 75.646) (width 1.1) (layer "B.Cu") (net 6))
 (segment (start 138.984 75.646) (end 143.51 75.646) (width 1.1) (layer "B.Cu") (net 6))
 (segment (start 125.227 74.168) (end 137.414 74.168) (width 1.1) (layer "B.Cu") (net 6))
 (segment (start 137.414 74.168) (end 138.938 75.692) (width 1.1) (layer "B.Cu") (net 6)))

